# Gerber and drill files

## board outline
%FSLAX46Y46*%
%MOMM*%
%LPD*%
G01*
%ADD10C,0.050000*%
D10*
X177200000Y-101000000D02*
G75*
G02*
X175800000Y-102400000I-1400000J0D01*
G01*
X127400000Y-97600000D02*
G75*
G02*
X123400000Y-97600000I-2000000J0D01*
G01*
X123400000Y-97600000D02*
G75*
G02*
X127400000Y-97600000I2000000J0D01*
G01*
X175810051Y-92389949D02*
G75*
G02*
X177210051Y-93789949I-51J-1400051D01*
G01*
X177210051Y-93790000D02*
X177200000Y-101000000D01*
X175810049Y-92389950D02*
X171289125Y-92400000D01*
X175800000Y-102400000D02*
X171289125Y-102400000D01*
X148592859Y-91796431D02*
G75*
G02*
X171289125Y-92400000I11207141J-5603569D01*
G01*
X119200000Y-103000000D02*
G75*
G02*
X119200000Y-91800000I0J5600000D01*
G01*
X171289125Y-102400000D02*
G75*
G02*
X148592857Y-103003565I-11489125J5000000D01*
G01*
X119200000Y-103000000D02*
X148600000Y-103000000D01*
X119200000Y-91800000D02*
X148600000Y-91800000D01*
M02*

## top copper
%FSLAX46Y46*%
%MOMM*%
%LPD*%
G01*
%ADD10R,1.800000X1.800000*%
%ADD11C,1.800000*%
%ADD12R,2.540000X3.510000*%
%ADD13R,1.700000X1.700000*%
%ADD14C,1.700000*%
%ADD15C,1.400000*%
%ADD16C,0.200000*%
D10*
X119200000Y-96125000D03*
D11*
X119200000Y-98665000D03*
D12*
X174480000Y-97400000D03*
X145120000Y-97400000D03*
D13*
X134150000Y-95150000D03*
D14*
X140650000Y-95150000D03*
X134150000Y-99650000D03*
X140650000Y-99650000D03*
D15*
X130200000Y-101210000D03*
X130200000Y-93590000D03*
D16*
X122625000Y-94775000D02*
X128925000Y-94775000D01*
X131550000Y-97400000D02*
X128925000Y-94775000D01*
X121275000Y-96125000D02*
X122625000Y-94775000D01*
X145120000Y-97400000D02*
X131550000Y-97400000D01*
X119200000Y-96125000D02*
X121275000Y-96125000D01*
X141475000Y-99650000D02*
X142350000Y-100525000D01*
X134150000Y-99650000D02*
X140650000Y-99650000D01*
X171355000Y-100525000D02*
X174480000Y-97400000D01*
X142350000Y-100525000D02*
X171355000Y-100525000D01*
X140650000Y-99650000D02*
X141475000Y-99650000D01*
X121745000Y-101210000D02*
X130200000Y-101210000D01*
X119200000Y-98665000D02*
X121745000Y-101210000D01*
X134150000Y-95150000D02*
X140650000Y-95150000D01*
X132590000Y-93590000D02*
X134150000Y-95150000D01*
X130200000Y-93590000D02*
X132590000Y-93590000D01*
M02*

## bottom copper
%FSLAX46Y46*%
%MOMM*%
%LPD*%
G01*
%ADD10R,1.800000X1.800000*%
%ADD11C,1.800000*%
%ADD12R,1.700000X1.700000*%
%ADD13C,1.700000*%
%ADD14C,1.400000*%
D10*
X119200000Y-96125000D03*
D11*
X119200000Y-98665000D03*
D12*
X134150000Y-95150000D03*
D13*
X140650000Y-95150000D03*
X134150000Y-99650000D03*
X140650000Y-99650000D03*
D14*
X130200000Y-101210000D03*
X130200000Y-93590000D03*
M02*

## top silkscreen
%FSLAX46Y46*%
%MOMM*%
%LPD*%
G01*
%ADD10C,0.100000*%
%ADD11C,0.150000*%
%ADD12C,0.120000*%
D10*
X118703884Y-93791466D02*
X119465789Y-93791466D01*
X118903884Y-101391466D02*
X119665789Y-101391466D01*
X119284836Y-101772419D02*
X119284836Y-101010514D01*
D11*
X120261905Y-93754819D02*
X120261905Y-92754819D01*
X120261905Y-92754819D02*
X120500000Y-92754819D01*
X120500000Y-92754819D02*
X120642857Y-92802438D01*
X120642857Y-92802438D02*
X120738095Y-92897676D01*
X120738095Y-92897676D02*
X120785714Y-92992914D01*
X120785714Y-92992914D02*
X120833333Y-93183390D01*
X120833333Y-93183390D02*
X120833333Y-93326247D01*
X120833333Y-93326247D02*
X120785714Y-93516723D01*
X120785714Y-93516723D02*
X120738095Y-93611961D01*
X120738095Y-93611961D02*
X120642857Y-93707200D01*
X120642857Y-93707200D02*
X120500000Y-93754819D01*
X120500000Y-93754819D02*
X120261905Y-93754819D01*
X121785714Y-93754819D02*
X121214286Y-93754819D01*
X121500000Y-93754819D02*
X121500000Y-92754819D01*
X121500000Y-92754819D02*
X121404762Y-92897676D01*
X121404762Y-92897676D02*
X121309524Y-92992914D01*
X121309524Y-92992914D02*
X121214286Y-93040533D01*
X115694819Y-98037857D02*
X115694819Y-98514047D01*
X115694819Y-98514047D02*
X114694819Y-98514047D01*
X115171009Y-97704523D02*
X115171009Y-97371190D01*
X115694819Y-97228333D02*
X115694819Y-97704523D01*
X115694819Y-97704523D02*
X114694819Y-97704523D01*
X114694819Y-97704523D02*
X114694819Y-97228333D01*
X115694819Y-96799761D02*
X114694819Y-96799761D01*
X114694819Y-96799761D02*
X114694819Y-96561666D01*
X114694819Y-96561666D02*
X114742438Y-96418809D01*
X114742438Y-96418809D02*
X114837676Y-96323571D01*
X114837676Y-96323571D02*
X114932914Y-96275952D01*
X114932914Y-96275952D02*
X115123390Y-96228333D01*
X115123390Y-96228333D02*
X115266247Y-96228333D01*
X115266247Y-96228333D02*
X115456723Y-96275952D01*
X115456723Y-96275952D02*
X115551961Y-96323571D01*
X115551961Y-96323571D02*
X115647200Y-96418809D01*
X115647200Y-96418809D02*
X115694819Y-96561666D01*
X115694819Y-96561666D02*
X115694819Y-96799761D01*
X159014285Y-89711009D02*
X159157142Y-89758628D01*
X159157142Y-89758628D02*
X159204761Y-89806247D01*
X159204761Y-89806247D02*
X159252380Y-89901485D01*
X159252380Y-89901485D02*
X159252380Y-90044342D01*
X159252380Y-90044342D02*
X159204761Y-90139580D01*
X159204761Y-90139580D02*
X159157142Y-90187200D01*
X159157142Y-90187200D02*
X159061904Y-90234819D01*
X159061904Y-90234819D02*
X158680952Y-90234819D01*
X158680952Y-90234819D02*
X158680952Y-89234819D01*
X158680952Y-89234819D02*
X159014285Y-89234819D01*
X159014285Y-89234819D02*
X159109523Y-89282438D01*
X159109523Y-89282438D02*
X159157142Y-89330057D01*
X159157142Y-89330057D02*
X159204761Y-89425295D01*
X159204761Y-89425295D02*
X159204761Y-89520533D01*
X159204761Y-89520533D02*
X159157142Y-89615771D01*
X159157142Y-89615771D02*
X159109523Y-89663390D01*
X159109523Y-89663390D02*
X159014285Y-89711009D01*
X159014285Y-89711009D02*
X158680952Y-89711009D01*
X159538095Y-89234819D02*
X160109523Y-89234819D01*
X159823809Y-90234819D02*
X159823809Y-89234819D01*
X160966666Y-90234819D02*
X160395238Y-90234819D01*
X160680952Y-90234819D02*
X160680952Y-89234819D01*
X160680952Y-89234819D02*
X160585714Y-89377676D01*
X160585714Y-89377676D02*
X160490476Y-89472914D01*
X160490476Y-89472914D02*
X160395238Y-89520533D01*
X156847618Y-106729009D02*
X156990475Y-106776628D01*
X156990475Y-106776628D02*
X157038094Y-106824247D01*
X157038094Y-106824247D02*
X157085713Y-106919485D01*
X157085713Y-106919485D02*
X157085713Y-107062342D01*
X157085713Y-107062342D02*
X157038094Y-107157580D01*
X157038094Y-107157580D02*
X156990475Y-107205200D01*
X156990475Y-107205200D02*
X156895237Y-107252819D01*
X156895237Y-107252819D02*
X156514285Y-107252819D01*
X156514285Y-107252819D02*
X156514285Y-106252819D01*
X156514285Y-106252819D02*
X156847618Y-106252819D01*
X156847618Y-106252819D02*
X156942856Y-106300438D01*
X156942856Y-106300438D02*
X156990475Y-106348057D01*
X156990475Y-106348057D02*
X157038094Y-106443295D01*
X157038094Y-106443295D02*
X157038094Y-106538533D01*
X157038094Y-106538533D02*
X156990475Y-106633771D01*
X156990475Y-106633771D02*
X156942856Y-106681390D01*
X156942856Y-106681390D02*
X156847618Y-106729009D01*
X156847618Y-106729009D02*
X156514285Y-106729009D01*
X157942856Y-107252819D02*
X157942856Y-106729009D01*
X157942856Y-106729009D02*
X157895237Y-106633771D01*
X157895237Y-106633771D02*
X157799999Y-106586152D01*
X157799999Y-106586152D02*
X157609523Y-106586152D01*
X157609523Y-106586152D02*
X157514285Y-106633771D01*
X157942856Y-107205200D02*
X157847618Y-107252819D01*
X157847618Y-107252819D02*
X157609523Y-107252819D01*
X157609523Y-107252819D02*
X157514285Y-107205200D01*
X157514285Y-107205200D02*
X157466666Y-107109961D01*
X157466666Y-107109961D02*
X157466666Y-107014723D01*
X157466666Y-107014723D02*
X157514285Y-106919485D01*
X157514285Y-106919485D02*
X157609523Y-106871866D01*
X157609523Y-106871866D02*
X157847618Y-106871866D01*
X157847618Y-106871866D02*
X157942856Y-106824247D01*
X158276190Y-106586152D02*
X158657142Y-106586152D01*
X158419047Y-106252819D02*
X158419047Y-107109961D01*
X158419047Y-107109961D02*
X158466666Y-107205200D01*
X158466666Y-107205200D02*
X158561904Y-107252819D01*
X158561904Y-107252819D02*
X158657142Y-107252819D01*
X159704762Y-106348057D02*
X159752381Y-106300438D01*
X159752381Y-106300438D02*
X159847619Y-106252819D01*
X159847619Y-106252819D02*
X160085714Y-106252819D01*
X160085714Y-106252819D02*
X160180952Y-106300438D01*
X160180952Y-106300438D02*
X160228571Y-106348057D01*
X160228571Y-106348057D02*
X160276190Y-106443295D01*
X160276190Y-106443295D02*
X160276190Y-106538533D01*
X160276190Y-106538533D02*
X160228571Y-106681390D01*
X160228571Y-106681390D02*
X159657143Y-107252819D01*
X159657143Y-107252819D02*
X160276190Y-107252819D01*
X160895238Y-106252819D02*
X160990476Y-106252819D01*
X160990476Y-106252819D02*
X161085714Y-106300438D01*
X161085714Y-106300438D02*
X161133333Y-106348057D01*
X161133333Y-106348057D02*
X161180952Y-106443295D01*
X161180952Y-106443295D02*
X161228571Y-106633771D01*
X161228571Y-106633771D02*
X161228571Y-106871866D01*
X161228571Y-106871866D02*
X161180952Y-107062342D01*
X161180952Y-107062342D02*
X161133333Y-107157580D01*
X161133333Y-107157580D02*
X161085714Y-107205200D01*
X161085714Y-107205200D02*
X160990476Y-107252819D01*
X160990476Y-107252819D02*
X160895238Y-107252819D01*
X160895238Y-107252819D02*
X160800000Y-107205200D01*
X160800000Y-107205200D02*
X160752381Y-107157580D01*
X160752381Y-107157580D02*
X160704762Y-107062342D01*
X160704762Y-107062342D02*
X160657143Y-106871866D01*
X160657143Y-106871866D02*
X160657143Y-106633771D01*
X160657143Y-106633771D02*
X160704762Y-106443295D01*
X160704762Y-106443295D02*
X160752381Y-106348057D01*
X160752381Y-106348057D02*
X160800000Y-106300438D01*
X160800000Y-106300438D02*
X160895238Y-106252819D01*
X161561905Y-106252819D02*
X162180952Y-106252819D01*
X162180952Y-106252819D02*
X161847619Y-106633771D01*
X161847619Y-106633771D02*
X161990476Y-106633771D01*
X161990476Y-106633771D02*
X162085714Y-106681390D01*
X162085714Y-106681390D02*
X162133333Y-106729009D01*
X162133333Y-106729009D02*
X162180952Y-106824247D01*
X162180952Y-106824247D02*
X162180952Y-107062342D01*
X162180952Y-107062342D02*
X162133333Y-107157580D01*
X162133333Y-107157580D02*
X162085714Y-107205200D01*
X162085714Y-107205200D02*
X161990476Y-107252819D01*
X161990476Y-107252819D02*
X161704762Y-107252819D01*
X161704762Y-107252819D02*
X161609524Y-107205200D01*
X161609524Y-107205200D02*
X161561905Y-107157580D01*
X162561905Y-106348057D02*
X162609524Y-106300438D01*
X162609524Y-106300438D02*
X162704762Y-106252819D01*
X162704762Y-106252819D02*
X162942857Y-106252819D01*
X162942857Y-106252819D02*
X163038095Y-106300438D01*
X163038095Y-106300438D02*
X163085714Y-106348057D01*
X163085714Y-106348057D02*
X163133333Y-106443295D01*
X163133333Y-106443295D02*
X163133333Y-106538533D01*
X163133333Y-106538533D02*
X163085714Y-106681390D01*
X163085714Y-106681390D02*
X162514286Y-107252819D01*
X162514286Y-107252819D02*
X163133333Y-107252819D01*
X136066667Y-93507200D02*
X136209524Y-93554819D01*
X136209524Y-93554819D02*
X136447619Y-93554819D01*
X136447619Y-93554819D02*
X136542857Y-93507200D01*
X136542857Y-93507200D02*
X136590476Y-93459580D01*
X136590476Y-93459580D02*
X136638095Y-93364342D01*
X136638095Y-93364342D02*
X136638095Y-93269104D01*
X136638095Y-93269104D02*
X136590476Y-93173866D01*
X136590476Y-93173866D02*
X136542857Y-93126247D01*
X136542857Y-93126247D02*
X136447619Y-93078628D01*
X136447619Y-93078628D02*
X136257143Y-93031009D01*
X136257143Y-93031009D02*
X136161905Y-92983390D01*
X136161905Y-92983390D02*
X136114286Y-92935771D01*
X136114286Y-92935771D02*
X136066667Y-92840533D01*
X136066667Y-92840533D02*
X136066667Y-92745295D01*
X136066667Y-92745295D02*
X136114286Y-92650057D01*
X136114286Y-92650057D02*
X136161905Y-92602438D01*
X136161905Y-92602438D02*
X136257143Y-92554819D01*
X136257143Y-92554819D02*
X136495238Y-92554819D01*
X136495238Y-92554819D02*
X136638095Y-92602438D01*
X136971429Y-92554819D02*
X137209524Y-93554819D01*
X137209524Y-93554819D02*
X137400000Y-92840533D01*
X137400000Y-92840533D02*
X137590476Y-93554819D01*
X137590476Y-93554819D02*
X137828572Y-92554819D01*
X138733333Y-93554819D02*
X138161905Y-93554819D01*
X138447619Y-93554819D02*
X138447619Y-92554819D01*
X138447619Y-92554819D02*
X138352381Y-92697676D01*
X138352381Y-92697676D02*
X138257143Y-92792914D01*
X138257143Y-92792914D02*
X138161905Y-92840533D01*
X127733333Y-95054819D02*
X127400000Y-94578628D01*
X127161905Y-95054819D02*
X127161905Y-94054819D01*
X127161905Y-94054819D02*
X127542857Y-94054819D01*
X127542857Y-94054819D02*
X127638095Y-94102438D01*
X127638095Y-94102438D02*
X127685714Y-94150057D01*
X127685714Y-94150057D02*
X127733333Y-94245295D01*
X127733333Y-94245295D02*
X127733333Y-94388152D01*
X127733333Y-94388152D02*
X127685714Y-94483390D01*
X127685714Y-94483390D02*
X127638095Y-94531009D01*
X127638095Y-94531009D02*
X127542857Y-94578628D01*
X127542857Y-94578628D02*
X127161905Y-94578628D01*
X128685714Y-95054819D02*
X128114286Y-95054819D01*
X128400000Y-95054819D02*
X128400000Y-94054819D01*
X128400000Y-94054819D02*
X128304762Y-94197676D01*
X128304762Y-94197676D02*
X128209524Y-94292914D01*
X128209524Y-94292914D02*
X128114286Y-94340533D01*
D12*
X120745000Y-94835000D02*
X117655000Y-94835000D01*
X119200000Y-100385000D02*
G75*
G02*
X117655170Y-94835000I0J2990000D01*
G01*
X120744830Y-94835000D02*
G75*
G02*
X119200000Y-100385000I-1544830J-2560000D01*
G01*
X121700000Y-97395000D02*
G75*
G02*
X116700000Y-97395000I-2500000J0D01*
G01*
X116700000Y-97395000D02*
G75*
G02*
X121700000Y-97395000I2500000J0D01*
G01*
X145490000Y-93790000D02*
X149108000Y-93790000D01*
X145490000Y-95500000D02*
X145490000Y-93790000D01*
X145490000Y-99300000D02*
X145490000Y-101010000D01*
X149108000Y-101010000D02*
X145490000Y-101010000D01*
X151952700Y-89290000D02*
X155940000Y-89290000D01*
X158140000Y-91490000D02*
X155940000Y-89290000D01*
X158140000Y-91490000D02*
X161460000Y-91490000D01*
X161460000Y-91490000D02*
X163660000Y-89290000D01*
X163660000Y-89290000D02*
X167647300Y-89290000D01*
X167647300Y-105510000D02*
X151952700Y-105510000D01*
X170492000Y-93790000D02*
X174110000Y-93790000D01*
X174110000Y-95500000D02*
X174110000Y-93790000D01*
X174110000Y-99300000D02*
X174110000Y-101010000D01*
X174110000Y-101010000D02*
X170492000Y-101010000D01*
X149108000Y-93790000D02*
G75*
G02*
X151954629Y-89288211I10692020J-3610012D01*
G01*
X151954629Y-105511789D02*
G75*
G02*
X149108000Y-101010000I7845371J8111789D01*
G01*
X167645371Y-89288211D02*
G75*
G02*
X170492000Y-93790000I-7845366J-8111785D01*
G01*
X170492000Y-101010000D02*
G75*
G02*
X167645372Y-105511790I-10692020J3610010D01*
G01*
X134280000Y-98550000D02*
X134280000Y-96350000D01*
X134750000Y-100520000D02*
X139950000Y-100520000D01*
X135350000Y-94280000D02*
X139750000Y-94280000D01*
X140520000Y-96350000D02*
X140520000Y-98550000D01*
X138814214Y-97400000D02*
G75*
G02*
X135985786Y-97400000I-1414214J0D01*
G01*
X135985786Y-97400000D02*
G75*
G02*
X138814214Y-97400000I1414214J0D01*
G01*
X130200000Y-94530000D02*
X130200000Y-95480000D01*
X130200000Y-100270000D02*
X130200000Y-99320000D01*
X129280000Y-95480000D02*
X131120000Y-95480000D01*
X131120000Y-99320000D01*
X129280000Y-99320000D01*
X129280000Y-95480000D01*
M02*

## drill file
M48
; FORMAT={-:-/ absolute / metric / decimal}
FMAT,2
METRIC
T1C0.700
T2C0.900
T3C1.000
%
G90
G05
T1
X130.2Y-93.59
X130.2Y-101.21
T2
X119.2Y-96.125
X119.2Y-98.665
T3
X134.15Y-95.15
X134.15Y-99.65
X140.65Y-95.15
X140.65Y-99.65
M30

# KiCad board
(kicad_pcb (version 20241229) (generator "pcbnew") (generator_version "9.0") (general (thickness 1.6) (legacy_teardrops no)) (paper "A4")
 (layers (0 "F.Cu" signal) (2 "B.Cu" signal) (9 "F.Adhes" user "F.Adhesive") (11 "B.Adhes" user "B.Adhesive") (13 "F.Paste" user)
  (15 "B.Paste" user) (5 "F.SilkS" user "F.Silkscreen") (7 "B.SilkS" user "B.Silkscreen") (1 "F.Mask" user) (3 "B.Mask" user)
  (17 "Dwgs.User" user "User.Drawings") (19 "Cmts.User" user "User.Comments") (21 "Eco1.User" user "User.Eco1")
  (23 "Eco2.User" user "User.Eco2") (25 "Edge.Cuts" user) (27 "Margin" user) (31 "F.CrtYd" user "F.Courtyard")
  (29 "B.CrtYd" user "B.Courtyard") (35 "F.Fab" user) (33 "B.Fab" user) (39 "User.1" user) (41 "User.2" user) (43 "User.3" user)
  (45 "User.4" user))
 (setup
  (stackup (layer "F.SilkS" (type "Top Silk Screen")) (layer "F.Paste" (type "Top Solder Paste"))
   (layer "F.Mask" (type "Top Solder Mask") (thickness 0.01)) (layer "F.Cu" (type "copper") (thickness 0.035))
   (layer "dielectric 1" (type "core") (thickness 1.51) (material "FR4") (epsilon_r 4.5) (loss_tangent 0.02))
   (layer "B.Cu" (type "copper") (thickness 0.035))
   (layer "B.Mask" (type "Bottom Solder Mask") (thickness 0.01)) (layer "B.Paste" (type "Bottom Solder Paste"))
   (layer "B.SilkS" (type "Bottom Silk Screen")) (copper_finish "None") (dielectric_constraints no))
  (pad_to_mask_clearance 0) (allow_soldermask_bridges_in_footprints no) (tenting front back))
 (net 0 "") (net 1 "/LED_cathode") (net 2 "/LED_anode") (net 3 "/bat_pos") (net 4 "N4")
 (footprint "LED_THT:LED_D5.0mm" (layer "F.Cu") (at 119.2 96.125 -90)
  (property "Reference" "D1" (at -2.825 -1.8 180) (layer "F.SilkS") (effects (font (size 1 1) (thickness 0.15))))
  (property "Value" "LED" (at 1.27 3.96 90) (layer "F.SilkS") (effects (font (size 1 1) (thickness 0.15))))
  (fp_line (start -1.29 -1.545) (end -1.29 1.545) (stroke (width 0.12) (type solid)) (layer "F.SilkS"))
  (fp_arc (start 4.26 0) (mid 2.071779 2.880495) (end -1.29 1.54483) (stroke (width 0.12) (type solid)) (layer "F.SilkS"))
  (fp_arc (start -1.29 -1.54483) (mid 2.071779 -2.880495) (end 4.26 0) (stroke (width 0.12) (type solid)) (layer "F.SilkS"))
  (fp_circle (center 1.27 0) (end 3.77 0) (stroke (width 0.12) (type solid)) (fill no) (layer "F.SilkS"))
  (pad "1" thru_hole rect (at 0 0 270) (size 1.8 1.8) (drill 0.9) (layers "*.Cu" "*.Mask") (remove_unused_layers no) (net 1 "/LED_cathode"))
  (pad "2" thru_hole circle (at 2.54 0 270) (size 1.8 1.8) (drill 0.9) (layers "*.Cu" "*.Mask") (remove_unused_layers no)
   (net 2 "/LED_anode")))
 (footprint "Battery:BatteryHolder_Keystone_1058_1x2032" (layer "F.Cu") (at 159.8 97.4 180)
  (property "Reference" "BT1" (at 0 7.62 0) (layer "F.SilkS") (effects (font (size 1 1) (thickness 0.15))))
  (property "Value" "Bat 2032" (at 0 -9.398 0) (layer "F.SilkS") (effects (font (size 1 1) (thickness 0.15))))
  (fp_line (start 14.31 3.61) (end 10.692 3.61) (stroke (width 0.12) (type solid)) (layer "F.SilkS"))
  (fp_line (start 14.31 1.9) (end 14.31 3.61) (stroke (width 0.12) (type solid)) (layer "F.SilkS"))
  (fp_line (start 14.31 -1.9) (end 14.31 -3.61) (stroke (width 0.12) (type solid)) (layer "F.SilkS"))
  (fp_line (start 10.692 -3.61) (end 14.31 -3.61) (stroke (width 0.12) (type solid)) (layer "F.SilkS"))
  (fp_line (start 7.8473 8.11) (end 3.86 8.11) (stroke (width 0.12) (type solid)) (layer "F.SilkS"))
  (fp_line (start 1.66 5.91) (end 3.86 8.11) (stroke (width 0.12) (type solid)) (layer "F.SilkS"))
  (fp_line (start 1.66 5.91) (end -1.66 5.91) (stroke (width 0.12) (type solid)) (layer "F.SilkS"))
  (fp_line (start -1.66 5.91) (end -3.86 8.11) (stroke (width 0.12) (type solid)) (layer "F.SilkS"))
  (fp_line (start -3.86 8.11) (end -7.8473 8.11) (stroke (width 0.12) (type solid)) (layer "F.SilkS"))
  (fp_line (start -7.8473 -8.11) (end 7.8473 -8.11) (stroke (width 0.12) (type solid)) (layer "F.SilkS"))
  (fp_line (start -10.692 3.61) (end -14.31 3.61) (stroke (width 0.12) (type solid)) (layer "F.SilkS"))
  (fp_line (start -14.31 1.9) (end -14.31 3.61) (stroke (width 0.12) (type solid)) (layer "F.SilkS"))
  (fp_line (start -14.31 -1.9) (end -14.31 -3.61) (stroke (width 0.12) (type solid)) (layer "F.SilkS"))
  (fp_line (start -14.31 -3.61) (end -10.692 -3.61) (stroke (width 0.12) (type solid)) (layer "F.SilkS"))
  (fp_arc (start 10.692 3.61) (mid 9.538084 6.031244) (end 7.845371 8.111789) (stroke (width 0.12) (type solid)) (layer "F.SilkS"))
  (fp_arc (start 7.845371 -8.111789) (mid 9.538085 -6.031244) (end 10.692 -3.61) (stroke (width 0.12) (type solid)) (layer "F.SilkS"))
  (fp_arc (start -7.845371 8.111789) (mid -9.538085 6.031244) (end -10.692 3.61) (stroke (width 0.12) (type solid)) (layer "F.SilkS"))
  (fp_arc (start -10.692 -3.61) (mid -9.538084 -6.031244) (end -7.845371 -8.111789) (stroke (width 0.12) (type solid)) (layer "F.SilkS"))
  (pad "1" smd rect (at -14.68 0 180) (size 2.54 3.51) (layers "F.Cu" "F.Mask" "F.Paste") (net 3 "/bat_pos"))
  (pad "2" smd rect (at 14.68 0 180) (size 2.54 3.51) (layers "F.Cu" "F.Mask" "F.Paste") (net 1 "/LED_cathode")))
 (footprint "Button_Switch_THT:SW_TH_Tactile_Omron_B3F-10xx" (layer "F.Cu") (at 134.15 95.15)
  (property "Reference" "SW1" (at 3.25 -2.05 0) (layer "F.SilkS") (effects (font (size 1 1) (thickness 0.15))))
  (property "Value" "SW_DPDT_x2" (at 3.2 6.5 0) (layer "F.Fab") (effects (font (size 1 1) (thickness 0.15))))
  (fp_line (start 0.13 3.4) (end 0.13 1.2) (stroke (width 0.12) (type solid)) (layer "F.SilkS"))
  (fp_line (start 0.6 5.37) (end 5.8 5.37) (stroke (width 0.12) (type solid)) (layer "F.SilkS"))
  (fp_line (start 1.2 -0.87) (end 5.6 -0.87) (stroke (width 0.12) (type solid)) (layer "F.SilkS"))
  (fp_line (start 6.37 1.2) (end 6.37 3.4) (stroke (width 0.12) (type solid)) (layer "F.SilkS"))
  (fp_circle (center 3.25 2.25) (end 4.25 3.25) (stroke (width 0.12) (type solid)) (fill no) (layer "F.SilkS"))
  (pad "1" thru_hole rect (at 0 0) (size 1.7 1.7) (drill 1) (layers "*.Cu" "*.Mask") (remove_unused_layers no) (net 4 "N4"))
  (pad "1" thru_hole circle (at 6.5 0) (size 1.7 1.7) (drill 1) (layers "*.Cu" "*.Mask") (remove_unused_layers no) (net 4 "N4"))
  (pad "2" thru_hole circle (at 0 4.5) (size 1.7 1.7) (drill 1) (layers "*.Cu" "*.Mask") (remove_unused_layers no) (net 3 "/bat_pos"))
  (pad "2" thru_hole circle (at 6.5 4.5) (size 1.7 1.7) (drill 1) (layers "*.Cu" "*.Mask") (remove_unused_layers no) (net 3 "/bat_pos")))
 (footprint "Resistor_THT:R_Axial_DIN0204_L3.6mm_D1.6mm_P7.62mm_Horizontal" (layer "F.Cu") (at 130.2 101.21 90)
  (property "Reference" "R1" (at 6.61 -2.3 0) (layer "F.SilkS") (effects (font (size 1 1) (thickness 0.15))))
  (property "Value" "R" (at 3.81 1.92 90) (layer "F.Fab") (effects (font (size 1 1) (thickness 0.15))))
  (fp_line (start 6.68 0) (end 5.73 0) (stroke (width 0.12) (type solid)) (layer "F.SilkS"))
  (fp_line (start 0.94 0) (end 1.89 0) (stroke (width 0.12) (type solid)) (layer "F.SilkS"))
  (fp_rect (start 1.89 -0.92) (end 5.73 0.92) (stroke (width 0.12) (type solid)) (fill no) (layer "F.SilkS"))
  (pad "1" thru_hole circle (at 0 0 90) (size 1.4 1.4) (drill 0.7) (layers "*.Cu" "*.Mask") (remove_unused_layers no) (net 2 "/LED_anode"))
  (pad "2" thru_hole circle (at 7.62 0 90) (size 1.4 1.4) (drill 0.7) (layers "*.Cu" "*.Mask") (remove_unused_layers no) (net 4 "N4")))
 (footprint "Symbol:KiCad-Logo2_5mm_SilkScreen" (layer "B.Cu") (at 160 94.4 180)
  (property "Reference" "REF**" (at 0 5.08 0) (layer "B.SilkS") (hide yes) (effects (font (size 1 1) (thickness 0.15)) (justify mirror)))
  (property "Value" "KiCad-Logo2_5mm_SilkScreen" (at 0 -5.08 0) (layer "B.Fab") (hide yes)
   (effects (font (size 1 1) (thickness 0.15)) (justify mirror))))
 (gr_arc (start 177.2 101) (mid 176.789949 101.989949) (end 175.8 102.4) (stroke (width 0.05) (type default)) (locked yes)
  (layer "Edge.Cuts"))
 (gr_circle (center 125.4 97.6) (end 127 98.8) (stroke (width 0.05) (type default)) (fill no) (layer "Edge.Cuts"))
 (gr_arc (start 175.810051 92.389949) (mid 176.8 92.8) (end 177.210051 93.789949) (stroke (width 0.05) (type default)) (locked yes)
  (layer "Edge.Cuts"))
 (gr_line (start 177.210051 93.79) (end 177.2 101) (stroke (width 0.05) (type default)) (locked yes) (layer "Edge.Cuts"))
 (gr_line (start 175.810049 92.38995) (end 171.289125 92.4) (stroke (width 0.05) (type default)) (locked yes) (layer "Edge.Cuts"))
 (gr_line (start 175.8 102.4) (end 171.289125 102.4) (stroke (width 0.05) (type default)) (locked yes) (layer "Edge.Cuts"))
 (gr_arc (start 148.592859 91.796431) (mid 160.133096 84.874464) (end 171.289125 92.4) (stroke (width 0.05) (type default)) (locked yes)
  (layer "Edge.Cuts"))
 (gr_arc (start 119.2 103) (mid 113.6 97.4) (end 119.2 91.8) (stroke (width 0.05) (type default)) (locked yes) (layer "Edge.Cuts"))
 (gr_arc (start 171.289125 102.4) (mid 160.133093 109.925536) (end 148.592857 103.003565) (stroke (width 0.05) (type default)) (locked yes)
  (layer "Edge.Cuts"))
 (gr_line (start 119.2 103) (end 148.6 103) (stroke (width 0.05) (type default)) (locked yes) (layer "Edge.Cuts"))
 (gr_line (start 119.2 91.8) (end 148.6 91.8) (stroke (width 0.05) (type default)) (locked yes) (layer "Edge.Cuts"))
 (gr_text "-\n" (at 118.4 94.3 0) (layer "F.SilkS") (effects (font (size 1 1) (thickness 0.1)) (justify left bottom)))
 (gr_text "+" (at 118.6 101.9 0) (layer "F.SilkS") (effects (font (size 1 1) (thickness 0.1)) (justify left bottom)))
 (segment (start 122.625 94.775) (end 128.925 94.775) (width 0.2) (layer "F.Cu") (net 1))
 (segment (start 131.55 97.4) (end 128.925 94.775) (width 0.2) (layer "F.Cu") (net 1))
 (segment (start 121.275 96.125) (end 122.625 94.775) (width 0.2) (layer "F.Cu") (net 1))
 (segment (start 145.12 97.4) (end 131.55 97.4) (width 0.2) (layer "F.Cu") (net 1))
 (segment (start 119.2 96.125) (end 121.275 96.125) (width 0.2) (layer "F.Cu") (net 1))
 (segment (start 141.475 99.65) (end 142.35 100.525) (width 0.2) (layer "F.Cu") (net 3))
 (segment (start 134.15 99.65) (end 140.65 99.65) (width 0.2) (layer "F.Cu") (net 3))
 (segment (start 171.355 100.525) (end 174.48 97.4) (width 0.2) (layer "F.Cu") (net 3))
 (segment (start 142.35 100.525) (end 171.355 100.525) (width 0.2) (layer "F.Cu") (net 3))
 (segment (start 140.65 99.65) (end 141.475 99.65) (width 0.2) (layer "F.Cu") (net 3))
 (segment (start 121.745 101.21) (end 130.2 101.21) (width 0.2) (layer "F.Cu") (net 2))
 (segment (start 119.2 98.665) (end 121.745 101.21) (width 0.2) (layer "F.Cu") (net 2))
 (segment (start 134.15 95.15) (end 140.65 95.15) (width 0.2) (layer "F.Cu") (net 4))
 (segment (start 132.59 93.59) (end 134.15 95.15) (width 0.2) (layer "F.Cu") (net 4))
 (segment (start 130.2 93.59) (end 132.59 93.59) (width 0.2) (layer "F.Cu") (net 4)))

